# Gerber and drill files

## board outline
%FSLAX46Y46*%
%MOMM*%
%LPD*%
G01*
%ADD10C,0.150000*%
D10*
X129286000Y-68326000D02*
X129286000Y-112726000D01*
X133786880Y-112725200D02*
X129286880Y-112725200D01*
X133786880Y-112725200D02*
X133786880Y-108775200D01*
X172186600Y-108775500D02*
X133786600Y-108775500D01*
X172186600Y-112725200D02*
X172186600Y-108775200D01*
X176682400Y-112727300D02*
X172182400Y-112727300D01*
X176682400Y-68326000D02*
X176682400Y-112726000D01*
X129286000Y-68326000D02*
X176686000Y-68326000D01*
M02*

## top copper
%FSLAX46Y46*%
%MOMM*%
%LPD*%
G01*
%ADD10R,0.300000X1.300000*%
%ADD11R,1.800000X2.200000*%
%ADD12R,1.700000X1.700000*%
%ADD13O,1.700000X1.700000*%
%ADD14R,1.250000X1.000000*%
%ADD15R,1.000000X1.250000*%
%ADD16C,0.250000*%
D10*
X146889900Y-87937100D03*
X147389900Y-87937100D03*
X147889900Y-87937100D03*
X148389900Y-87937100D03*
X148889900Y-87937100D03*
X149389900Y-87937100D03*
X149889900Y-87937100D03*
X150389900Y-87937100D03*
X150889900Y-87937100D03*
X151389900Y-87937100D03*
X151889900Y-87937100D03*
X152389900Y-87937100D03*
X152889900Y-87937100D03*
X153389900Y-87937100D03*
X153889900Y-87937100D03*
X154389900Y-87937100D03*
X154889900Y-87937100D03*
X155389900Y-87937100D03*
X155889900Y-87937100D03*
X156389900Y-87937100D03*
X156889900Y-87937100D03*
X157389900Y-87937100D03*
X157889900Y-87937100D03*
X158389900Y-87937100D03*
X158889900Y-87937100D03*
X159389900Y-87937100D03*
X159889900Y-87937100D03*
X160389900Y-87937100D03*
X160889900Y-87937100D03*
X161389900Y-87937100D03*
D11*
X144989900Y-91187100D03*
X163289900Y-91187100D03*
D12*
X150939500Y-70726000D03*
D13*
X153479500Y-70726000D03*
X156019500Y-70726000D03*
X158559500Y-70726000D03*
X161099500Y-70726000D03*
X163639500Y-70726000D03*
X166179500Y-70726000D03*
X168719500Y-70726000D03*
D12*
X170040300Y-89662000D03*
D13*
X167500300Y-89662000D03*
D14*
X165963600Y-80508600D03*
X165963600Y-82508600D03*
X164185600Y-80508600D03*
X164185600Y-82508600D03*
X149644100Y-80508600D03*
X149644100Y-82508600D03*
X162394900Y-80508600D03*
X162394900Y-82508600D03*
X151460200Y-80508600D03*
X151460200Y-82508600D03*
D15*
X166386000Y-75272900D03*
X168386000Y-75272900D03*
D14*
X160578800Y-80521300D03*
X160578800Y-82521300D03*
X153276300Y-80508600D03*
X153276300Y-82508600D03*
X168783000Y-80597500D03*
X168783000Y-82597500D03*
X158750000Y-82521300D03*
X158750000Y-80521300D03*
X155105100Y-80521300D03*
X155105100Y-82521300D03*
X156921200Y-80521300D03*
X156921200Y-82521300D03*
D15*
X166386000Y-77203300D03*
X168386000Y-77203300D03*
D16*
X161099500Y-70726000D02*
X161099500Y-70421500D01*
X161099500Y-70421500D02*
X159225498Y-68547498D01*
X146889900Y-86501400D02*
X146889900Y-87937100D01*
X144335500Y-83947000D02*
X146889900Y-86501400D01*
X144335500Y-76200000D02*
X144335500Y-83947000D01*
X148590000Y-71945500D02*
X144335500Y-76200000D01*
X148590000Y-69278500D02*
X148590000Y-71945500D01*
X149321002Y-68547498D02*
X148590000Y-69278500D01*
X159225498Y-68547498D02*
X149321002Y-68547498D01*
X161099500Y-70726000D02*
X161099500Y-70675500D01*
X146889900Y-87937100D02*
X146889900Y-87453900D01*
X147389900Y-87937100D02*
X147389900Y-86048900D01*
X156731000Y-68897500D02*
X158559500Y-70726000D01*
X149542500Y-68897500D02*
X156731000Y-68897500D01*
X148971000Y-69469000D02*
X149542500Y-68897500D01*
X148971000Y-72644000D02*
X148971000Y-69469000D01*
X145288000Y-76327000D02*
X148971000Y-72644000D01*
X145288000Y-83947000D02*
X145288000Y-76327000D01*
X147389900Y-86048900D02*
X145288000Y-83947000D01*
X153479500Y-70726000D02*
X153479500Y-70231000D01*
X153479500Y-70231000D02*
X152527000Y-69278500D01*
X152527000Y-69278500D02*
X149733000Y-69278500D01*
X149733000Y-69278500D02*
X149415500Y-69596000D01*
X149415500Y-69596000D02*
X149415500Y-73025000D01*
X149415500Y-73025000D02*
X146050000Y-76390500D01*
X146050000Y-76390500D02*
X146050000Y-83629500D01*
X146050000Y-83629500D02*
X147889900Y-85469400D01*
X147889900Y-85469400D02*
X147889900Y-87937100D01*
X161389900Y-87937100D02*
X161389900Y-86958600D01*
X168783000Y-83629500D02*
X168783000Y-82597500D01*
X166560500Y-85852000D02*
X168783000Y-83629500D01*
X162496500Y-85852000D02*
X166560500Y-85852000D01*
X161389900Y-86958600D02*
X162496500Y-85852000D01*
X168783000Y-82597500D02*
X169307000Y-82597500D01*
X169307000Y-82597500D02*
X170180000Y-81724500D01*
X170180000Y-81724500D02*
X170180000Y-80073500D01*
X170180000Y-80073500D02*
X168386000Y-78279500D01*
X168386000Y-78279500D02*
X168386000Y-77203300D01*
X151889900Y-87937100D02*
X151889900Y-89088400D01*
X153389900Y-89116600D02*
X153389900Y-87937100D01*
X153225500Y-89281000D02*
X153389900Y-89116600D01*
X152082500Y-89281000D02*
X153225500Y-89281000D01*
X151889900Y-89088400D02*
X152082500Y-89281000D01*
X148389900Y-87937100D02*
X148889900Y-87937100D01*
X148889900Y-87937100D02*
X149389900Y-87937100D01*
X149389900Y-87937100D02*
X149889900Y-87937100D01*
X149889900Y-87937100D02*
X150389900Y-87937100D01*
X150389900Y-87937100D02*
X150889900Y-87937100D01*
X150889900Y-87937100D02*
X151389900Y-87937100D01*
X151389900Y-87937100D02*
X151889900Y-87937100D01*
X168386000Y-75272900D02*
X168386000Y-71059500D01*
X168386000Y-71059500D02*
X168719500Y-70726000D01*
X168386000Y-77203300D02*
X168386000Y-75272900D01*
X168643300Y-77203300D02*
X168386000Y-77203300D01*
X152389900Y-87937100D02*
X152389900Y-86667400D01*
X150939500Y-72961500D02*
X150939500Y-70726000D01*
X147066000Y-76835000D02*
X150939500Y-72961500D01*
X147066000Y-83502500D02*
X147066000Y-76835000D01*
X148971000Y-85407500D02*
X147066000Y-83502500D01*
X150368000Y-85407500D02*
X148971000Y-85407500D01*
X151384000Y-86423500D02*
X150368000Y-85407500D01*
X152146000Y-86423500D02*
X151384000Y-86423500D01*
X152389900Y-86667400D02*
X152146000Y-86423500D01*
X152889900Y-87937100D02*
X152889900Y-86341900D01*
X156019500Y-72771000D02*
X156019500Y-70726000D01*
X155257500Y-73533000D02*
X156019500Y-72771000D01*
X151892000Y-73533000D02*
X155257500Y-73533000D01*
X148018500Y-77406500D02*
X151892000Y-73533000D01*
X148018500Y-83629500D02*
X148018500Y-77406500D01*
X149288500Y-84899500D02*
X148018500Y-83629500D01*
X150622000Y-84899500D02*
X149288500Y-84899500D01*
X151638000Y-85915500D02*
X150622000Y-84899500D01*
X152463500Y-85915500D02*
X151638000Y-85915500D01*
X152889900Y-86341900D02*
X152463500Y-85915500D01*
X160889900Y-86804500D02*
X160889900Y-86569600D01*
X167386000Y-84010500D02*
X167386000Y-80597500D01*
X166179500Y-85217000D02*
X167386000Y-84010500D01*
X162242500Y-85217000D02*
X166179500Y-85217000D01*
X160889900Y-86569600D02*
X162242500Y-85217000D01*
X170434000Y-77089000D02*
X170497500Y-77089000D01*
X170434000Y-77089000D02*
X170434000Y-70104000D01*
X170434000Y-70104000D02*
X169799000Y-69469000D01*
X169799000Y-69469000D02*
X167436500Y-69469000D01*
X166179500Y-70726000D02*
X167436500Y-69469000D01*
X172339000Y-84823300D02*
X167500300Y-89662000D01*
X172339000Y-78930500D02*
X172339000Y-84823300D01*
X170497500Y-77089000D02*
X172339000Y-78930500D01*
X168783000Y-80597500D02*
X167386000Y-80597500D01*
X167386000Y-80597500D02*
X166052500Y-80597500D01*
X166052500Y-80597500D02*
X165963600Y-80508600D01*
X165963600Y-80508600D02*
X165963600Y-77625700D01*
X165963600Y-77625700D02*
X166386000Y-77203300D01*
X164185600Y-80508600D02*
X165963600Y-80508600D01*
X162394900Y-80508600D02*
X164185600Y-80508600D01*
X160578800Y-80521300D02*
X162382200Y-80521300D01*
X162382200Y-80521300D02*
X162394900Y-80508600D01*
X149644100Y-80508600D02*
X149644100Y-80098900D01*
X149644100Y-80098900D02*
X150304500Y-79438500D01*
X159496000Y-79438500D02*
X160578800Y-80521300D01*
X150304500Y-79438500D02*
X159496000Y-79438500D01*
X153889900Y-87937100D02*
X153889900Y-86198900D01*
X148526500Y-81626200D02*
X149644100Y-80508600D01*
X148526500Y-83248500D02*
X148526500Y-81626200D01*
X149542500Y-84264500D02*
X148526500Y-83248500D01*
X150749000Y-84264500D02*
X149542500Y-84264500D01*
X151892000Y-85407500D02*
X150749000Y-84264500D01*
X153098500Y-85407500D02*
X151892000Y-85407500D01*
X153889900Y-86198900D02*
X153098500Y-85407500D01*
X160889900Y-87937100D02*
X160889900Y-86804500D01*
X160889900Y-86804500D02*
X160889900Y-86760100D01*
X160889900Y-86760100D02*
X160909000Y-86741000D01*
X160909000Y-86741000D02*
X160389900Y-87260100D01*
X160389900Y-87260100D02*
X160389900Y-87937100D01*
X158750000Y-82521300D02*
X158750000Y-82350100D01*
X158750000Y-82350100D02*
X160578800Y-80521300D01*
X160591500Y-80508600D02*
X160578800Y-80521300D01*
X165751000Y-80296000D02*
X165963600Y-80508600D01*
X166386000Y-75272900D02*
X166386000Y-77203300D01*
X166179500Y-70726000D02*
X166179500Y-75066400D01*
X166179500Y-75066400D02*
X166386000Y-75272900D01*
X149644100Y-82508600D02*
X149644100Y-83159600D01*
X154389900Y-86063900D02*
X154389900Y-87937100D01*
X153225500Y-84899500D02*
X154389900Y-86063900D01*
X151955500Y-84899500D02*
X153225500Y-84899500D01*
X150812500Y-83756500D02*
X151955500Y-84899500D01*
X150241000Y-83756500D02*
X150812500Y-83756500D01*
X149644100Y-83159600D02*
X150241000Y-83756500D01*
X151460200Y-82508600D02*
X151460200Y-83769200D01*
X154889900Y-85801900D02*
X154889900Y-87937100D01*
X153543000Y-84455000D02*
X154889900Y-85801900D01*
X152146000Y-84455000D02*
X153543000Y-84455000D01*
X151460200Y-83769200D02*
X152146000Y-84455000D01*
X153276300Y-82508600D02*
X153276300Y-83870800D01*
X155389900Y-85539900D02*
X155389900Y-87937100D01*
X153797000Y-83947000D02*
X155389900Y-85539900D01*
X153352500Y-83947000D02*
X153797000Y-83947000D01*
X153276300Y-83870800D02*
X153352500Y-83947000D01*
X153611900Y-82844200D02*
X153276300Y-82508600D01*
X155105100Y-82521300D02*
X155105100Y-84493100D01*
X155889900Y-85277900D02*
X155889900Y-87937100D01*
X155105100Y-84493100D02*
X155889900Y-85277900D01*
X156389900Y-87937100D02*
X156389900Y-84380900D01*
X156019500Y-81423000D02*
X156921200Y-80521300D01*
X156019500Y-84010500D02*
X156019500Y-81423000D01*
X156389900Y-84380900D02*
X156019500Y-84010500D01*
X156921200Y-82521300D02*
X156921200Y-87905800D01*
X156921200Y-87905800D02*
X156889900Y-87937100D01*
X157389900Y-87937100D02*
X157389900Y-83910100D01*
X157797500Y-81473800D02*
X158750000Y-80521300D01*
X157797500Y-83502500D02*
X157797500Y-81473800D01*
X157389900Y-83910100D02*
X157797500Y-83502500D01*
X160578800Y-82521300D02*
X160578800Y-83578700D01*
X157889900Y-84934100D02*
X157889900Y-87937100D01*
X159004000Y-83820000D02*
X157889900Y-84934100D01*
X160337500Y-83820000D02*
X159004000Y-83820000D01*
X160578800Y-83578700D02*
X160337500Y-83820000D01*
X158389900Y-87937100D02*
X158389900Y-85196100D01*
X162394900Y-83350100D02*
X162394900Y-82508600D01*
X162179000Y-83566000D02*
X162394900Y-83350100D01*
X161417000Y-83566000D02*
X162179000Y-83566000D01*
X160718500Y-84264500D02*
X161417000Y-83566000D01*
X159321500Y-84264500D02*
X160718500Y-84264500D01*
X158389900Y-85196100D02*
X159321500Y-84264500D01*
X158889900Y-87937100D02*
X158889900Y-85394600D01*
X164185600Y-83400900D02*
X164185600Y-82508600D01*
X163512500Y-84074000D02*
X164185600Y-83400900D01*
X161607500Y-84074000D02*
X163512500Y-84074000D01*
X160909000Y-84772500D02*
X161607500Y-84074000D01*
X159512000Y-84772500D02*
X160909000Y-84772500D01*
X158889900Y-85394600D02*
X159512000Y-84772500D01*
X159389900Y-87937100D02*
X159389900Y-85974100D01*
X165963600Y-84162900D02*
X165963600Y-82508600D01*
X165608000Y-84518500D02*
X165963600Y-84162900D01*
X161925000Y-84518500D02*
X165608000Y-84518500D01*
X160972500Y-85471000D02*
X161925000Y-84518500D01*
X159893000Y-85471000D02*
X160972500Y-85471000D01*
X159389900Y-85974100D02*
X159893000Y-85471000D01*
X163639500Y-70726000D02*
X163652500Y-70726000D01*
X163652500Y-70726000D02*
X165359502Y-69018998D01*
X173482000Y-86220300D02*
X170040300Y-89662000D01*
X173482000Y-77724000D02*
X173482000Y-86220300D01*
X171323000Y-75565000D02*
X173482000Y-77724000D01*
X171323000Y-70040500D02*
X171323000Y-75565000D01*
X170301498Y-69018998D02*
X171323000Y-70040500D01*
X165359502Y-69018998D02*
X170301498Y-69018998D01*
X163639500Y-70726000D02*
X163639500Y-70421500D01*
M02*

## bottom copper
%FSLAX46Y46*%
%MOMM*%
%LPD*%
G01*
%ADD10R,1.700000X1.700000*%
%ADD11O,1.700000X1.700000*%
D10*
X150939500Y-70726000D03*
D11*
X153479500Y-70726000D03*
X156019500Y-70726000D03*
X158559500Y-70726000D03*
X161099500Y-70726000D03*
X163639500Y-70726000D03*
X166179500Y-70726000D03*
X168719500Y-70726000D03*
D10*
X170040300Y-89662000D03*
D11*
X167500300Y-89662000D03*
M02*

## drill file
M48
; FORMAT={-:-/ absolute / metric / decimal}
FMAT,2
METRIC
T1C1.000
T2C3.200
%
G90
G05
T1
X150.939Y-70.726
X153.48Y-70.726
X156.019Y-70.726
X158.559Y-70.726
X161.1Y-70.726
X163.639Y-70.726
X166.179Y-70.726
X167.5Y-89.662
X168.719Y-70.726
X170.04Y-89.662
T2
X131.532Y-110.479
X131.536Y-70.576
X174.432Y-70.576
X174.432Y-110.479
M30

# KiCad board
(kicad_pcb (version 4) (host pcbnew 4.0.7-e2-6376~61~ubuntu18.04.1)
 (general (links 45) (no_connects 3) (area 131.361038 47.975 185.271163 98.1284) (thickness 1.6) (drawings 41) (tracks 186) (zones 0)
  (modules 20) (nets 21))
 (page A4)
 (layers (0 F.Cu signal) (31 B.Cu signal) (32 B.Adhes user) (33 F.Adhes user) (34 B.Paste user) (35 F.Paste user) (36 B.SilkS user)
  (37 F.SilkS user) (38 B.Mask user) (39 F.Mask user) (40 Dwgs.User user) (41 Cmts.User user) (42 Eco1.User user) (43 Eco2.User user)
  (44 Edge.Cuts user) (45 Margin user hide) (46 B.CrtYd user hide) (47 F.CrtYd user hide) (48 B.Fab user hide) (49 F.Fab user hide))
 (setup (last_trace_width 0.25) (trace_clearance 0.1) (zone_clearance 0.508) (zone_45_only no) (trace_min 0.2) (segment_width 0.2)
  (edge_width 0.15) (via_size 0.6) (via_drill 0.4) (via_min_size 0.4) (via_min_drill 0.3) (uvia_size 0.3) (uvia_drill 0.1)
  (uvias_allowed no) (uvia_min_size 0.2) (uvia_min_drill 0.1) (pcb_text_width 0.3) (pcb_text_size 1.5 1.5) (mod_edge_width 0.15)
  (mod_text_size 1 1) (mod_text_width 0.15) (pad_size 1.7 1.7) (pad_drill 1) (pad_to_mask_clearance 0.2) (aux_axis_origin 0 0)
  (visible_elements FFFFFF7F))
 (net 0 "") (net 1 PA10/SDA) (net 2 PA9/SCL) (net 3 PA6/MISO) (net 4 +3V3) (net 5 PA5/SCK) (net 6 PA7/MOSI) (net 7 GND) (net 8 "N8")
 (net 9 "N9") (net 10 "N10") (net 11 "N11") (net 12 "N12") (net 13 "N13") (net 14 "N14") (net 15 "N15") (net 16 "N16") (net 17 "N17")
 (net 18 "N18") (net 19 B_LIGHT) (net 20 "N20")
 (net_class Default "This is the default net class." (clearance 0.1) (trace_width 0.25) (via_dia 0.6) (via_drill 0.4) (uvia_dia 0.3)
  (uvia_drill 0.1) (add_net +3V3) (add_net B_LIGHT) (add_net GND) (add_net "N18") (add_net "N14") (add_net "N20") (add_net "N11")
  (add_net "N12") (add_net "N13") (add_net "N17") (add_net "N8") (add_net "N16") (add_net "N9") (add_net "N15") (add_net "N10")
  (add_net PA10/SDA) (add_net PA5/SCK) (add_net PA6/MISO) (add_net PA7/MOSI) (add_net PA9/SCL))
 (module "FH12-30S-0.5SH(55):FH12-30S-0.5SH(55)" (layer F.Cu) (at 154.1399 88.4301)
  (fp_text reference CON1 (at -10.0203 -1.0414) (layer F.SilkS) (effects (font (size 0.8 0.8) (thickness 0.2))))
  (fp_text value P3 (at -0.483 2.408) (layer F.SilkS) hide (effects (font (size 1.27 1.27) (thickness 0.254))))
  (pad 1 smd rect (at -7.25 -0.493) (size 0.3 1.3) (layers F.Cu F.Paste F.Mask) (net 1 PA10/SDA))
  (pad 2 smd rect (at -6.75 -0.493) (size 0.3 1.3) (layers F.Cu F.Paste F.Mask) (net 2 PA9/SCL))
  (pad 3 smd rect (at -6.25 -0.493) (size 0.3 1.3) (layers F.Cu F.Paste F.Mask) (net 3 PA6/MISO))
  (pad 4 smd rect (at -5.75 -0.493) (size 0.3 1.3) (layers F.Cu F.Paste F.Mask) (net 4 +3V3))
  (pad 5 smd rect (at -5.25 -0.493) (size 0.3 1.3) (layers F.Cu F.Paste F.Mask) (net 4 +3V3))
  (pad 6 smd rect (at -4.75 -0.493) (size 0.3 1.3) (layers F.Cu F.Paste F.Mask) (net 4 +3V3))
  (pad 7 smd rect (at -4.25 -0.493) (size 0.3 1.3) (layers F.Cu F.Paste F.Mask) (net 4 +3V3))
  (pad 8 smd rect (at -3.75 -0.493) (size 0.3 1.3) (layers F.Cu F.Paste F.Mask) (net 4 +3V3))
  (pad 9 smd rect (at -3.25 -0.493) (size 0.3 1.3) (layers F.Cu F.Paste F.Mask) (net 4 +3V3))
  (pad 10 smd rect (at -2.75 -0.493) (size 0.3 1.3) (layers F.Cu F.Paste F.Mask) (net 4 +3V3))
  (pad 11 smd rect (at -2.25 -0.493) (size 0.3 1.3) (layers F.Cu F.Paste F.Mask) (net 4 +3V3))
  (pad 12 smd rect (at -1.75 -0.493) (size 0.3 1.3) (layers F.Cu F.Paste F.Mask) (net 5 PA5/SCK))
  (pad 13 smd rect (at -1.25 -0.493) (size 0.3 1.3) (layers F.Cu F.Paste F.Mask) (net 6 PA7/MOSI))
  (pad 14 smd rect (at -0.75 -0.493) (size 0.3 1.3) (layers F.Cu F.Paste F.Mask) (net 4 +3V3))
  (pad 15 smd rect (at -0.25 -0.493) (size 0.3 1.3) (layers F.Cu F.Paste F.Mask) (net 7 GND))
  (pad 16 smd rect (at 0.25 -0.493) (size 0.3 1.3) (layers F.Cu F.Paste F.Mask) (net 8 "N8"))
  (pad 17 smd rect (at 0.75 -0.493) (size 0.3 1.3) (layers F.Cu F.Paste F.Mask) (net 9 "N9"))
  (pad 18 smd rect (at 1.25 -0.493) (size 0.3 1.3) (layers F.Cu F.Paste F.Mask) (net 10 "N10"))
  (pad 19 smd rect (at 1.75 -0.493) (size 0.3 1.3) (layers F.Cu F.Paste F.Mask) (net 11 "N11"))
  (pad 20 smd rect (at 2.25 -0.493) (size 0.3 1.3) (layers F.Cu F.Paste F.Mask) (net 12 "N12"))
  (pad 21 smd rect (at 2.75 -0.493) (size 0.3 1.3) (layers F.Cu F.Paste F.Mask) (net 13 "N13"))
  (pad 22 smd rect (at 3.25 -0.493) (size 0.3 1.3) (layers F.Cu F.Paste F.Mask) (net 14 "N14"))
  (pad 23 smd rect (at 3.75 -0.493) (size 0.3 1.3) (layers F.Cu F.Paste F.Mask) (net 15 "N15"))
  (pad 24 smd rect (at 4.25 -0.493) (size 0.3 1.3) (layers F.Cu F.Paste F.Mask) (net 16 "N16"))
  (pad 25 smd rect (at 4.75 -0.493) (size 0.3 1.3) (layers F.Cu F.Paste F.Mask) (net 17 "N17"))
  (pad 26 smd rect (at 5.25 -0.493) (size 0.3 1.3) (layers F.Cu F.Paste F.Mask) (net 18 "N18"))
  (pad 27 smd rect (at 5.75 -0.493) (size 0.3 1.3) (layers F.Cu F.Paste F.Mask))
  (pad 28 smd rect (at 6.25 -0.493) (size 0.3 1.3) (layers F.Cu F.Paste F.Mask) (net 7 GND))
  (pad 29 smd rect (at 6.75 -0.493) (size 0.3 1.3) (layers F.Cu F.Paste F.Mask) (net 7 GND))
  (pad 30 smd rect (at 7.25 -0.493) (size 0.3 1.3) (layers F.Cu F.Paste F.Mask) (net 4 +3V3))
  (pad 31 smd rect (at -9.15 2.757) (size 1.8 2.2) (layers F.Cu F.Paste F.Mask))
  (pad 32 smd rect (at 9.15 2.757) (size 1.8 2.2) (layers F.Cu F.Paste F.Mask)))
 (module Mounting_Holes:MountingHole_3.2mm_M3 (layer F.Cu) (at 174.4324 110.4794)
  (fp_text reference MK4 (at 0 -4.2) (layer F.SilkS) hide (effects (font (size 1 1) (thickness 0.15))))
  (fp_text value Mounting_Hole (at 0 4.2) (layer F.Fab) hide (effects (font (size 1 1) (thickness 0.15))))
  (pad 1 np_thru_hole circle (at 0 0) (size 3.2 3.2) (drill 3.2) (layers *.Cu *.Mask)))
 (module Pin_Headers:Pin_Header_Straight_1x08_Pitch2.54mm (layer F.Cu) (at 150.9395 70.726 90)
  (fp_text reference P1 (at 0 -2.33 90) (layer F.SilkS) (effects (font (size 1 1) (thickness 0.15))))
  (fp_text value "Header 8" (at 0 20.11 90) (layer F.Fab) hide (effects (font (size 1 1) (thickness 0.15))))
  (pad 1 thru_hole rect (at 0 0 90) (size 1.7 1.7) (drill 1) (layers *.Cu *.Mask) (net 5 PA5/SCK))
  (pad 2 thru_hole oval (at 0 2.54 90) (size 1.7 1.7) (drill 1) (layers *.Cu *.Mask) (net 3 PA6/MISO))
  (pad 3 thru_hole oval (at 0 5.08 90) (size 1.7 1.7) (drill 1) (layers *.Cu *.Mask) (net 6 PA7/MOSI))
  (pad 4 thru_hole oval (at 0 7.62 90) (size 1.7 1.7) (drill 1) (layers *.Cu *.Mask) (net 2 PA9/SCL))
  (pad 5 thru_hole oval (at 0 10.16 90) (size 1.7 1.7) (drill 1) (layers *.Cu *.Mask) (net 1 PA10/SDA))
  (pad 6 thru_hole oval (at 0 12.7 90) (size 1.7 1.7) (drill 1) (layers *.Cu *.Mask) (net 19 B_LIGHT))
  (pad 7 thru_hole oval (at 0 15.24 90) (size 1.7 1.7) (drill 1) (layers *.Cu *.Mask) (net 7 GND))
  (pad 8 thru_hole oval (at 0 17.78 90) (size 1.7 1.7) (drill 1) (layers *.Cu *.Mask) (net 4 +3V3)))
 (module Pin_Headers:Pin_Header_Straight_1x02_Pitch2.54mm (layer F.Cu) (at 170.0403 89.662 270)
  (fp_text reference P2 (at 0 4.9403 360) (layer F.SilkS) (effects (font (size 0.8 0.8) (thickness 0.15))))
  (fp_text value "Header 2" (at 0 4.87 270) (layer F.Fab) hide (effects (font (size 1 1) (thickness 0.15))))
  (pad 1 thru_hole rect (at 0 0 270) (size 1.7 1.7) (drill 1) (layers *.Cu *.Mask) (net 19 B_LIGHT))
  (pad 2 thru_hole oval (at 0 2.54 270) (size 1.7 1.7) (drill 1) (layers *.Cu *.Mask) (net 7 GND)))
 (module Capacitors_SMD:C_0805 (layer F.Cu) (at 165.9636 81.5086 270)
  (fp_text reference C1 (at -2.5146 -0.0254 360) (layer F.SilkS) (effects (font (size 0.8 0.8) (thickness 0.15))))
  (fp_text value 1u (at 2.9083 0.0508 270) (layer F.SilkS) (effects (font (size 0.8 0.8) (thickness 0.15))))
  (pad 1 smd rect (at -1 0 270) (size 1 1.25) (layers F.Cu F.Paste F.Mask) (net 7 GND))
  (pad 2 smd rect (at 1 0 270) (size 1 1.25) (layers F.Cu F.Paste F.Mask) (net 18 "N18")))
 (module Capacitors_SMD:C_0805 (layer F.Cu) (at 164.1856 81.5086 270)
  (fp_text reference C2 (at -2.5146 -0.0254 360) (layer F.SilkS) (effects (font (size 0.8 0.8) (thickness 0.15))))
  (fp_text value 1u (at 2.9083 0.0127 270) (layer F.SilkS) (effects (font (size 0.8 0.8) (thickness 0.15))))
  (pad 1 smd rect (at -1 0 270) (size 1 1.25) (layers F.Cu F.Paste F.Mask) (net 7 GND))
  (pad 2 smd rect (at 1 0 270) (size 1 1.25) (layers F.Cu F.Paste F.Mask) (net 17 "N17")))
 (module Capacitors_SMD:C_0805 (layer F.Cu) (at 149.6441 81.5086 270)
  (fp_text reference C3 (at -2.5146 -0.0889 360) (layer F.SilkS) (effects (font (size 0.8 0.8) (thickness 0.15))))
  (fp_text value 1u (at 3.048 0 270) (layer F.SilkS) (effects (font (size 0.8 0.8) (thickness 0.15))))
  (pad 1 smd rect (at -1 0 270) (size 1 1.25) (layers F.Cu F.Paste F.Mask) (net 7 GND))
  (pad 2 smd rect (at 1 0 270) (size 1 1.25) (layers F.Cu F.Paste F.Mask) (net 8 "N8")))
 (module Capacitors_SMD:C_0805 (layer F.Cu) (at 162.3949 81.5086 270)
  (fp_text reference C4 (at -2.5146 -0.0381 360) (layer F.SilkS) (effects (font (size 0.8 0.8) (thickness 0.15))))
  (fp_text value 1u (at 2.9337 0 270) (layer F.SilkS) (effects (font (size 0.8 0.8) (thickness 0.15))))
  (pad 1 smd rect (at -1 0 270) (size 1 1.25) (layers F.Cu F.Paste F.Mask) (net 7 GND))
  (pad 2 smd rect (at 1 0 270) (size 1 1.25) (layers F.Cu F.Paste F.Mask) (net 16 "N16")))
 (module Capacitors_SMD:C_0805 (layer F.Cu) (at 151.4602 81.5086 270)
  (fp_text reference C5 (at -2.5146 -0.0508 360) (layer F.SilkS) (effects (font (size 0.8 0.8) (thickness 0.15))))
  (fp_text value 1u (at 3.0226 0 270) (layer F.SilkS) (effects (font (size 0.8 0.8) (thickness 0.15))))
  (pad 1 smd rect (at -1 0 270) (size 1 1.25) (layers F.Cu F.Paste F.Mask) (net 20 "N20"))
  (pad 2 smd rect (at 1 0 270) (size 1 1.25) (layers F.Cu F.Paste F.Mask) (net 9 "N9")))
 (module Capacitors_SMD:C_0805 (layer F.Cu) (at 167.386 75.2729)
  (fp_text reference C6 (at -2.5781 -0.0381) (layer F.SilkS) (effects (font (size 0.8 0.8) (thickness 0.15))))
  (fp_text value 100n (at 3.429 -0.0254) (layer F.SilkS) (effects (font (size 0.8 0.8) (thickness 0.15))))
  (pad 1 smd rect (at -1 0) (size 1 1.25) (layers F.Cu F.Paste F.Mask) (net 7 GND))
  (pad 2 smd rect (at 1 0) (size 1 1.25) (layers F.Cu F.Paste F.Mask) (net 4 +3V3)))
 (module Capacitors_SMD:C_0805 (layer F.Cu) (at 160.5788 81.5213 270)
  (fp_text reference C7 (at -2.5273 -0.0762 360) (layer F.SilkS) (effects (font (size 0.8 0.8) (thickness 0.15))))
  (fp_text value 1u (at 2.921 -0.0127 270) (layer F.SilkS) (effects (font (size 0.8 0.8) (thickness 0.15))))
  (pad 1 smd rect (at -1 0 270) (size 1 1.25) (layers F.Cu F.Paste F.Mask) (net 7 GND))
  (pad 2 smd rect (at 1 0 270) (size 1 1.25) (layers F.Cu F.Paste F.Mask) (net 15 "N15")))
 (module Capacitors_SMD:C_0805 (layer F.Cu) (at 153.2763 81.5086 270)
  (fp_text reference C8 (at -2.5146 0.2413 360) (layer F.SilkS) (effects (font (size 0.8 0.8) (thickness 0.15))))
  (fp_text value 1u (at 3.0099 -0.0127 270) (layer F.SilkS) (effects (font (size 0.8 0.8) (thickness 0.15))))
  (pad 1 smd rect (at -1 0 270) (size 1 1.25) (layers F.Cu F.Paste F.Mask) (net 20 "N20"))
  (pad 2 smd rect (at 1 0 270) (size 1 1.25) (layers F.Cu F.Paste F.Mask) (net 10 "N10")))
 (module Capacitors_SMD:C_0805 (layer F.Cu) (at 168.783 81.5975 270)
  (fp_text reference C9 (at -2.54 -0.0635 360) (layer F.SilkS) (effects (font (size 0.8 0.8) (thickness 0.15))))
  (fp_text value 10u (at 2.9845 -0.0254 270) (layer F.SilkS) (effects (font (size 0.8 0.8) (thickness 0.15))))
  (pad 1 smd rect (at -1 0 270) (size 1 1.25) (layers F.Cu F.Paste F.Mask) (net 7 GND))
  (pad 2 smd rect (at 1 0 270) (size 1 1.25) (layers F.Cu F.Paste F.Mask) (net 4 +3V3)))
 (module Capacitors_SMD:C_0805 (layer F.Cu) (at 158.75 81.5213 90)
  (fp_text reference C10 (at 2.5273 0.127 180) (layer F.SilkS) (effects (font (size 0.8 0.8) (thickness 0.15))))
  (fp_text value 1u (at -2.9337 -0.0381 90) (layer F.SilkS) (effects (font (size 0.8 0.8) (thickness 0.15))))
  (pad 1 smd rect (at -1 0 90) (size 1 1.25) (layers F.Cu F.Paste F.Mask) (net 7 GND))
  (pad 2 smd rect (at 1 0 90) (size 1 1.25) (layers F.Cu F.Paste F.Mask) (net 14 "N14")))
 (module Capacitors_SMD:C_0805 (layer F.Cu) (at 155.1051 81.5213 270)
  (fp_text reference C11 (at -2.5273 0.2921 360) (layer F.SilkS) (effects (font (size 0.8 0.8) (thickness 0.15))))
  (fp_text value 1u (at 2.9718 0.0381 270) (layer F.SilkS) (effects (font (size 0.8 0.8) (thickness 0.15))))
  (pad 1 smd rect (at -1 0 270) (size 1 1.25) (layers F.Cu F.Paste F.Mask) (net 20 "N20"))
  (pad 2 smd rect (at 1 0 270) (size 1 1.25) (layers F.Cu F.Paste F.Mask) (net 11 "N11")))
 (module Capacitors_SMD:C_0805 (layer F.Cu) (at 156.9212 81.5213 270)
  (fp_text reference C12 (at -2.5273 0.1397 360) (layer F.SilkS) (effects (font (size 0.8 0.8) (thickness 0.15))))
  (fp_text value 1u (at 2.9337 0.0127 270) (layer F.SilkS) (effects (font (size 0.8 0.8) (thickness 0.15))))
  (pad 1 smd rect (at -1 0 270) (size 1 1.25) (layers F.Cu F.Paste F.Mask) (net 12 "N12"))
  (pad 2 smd rect (at 1 0 270) (size 1 1.25) (layers F.Cu F.Paste F.Mask) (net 13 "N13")))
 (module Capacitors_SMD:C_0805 (layer F.Cu) (at 167.386 77.2033)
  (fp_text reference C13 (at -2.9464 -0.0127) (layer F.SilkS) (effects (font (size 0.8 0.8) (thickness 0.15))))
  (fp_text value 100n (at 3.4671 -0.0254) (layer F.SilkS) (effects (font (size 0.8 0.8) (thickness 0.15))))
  (pad 1 smd rect (at -1 0) (size 1 1.25) (layers F.Cu F.Paste F.Mask) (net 7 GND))
  (pad 2 smd rect (at 1 0) (size 1 1.25) (layers F.Cu F.Paste F.Mask) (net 4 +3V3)))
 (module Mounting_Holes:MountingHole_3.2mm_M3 (layer F.Cu) (at 131.536 70.576)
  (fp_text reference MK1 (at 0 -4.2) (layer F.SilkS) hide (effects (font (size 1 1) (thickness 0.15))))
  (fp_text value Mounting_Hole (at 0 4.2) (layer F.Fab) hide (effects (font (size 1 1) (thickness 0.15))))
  (pad 1 np_thru_hole circle (at 0 0) (size 3.2 3.2) (drill 3.2) (layers *.Cu *.Mask)))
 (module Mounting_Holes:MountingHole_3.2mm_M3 (layer F.Cu) (at 174.4324 70.576)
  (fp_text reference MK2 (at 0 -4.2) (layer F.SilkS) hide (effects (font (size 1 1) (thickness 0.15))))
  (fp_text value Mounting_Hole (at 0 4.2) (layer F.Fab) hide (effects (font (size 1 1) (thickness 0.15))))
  (pad 1 np_thru_hole circle (at 0 0) (size 3.2 3.2) (drill 3.2) (layers *.Cu *.Mask)))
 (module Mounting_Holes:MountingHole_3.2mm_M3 (layer F.Cu) (at 131.5318 110.4794)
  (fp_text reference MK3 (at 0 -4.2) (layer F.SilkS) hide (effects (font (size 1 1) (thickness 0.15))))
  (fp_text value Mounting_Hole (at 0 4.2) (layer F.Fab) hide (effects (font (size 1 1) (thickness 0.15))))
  (pad 1 np_thru_hole circle (at 0 0) (size 3.2 3.2) (drill 3.2) (layers *.Cu *.Mask)))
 (gr_line (start 129.286 68.326) (end 129.286 112.726) (angle 90) (layer Edge.Cuts) (width 0.15))
 (gr_line (start 133.78688 112.7252) (end 129.28688 112.7252) (angle 90) (layer Edge.Cuts) (width 0.15))
 (gr_line (start 133.78688 112.7252) (end 133.78688 108.7752) (angle 90) (layer Edge.Cuts) (width 0.15))
 (gr_line (start 172.1866 108.7755) (end 133.7866 108.7755) (angle 90) (layer Edge.Cuts) (width 0.15))
 (gr_line (start 172.1866 112.7252) (end 172.1866 108.7752) (angle 90) (layer Edge.Cuts) (width 0.15))
 (gr_line (start 176.6824 112.7273) (end 172.1824 112.7273) (angle 90) (layer Edge.Cuts) (width 0.15))
 (gr_line (start 176.6824 68.326) (end 176.6824 112.726) (angle 90) (layer Edge.Cuts) (width 0.15))
 (gr_line (start 129.286 68.326) (end 176.686 68.326) (angle 90) (layer Edge.Cuts) (width 0.15))
 (segment (start 161.0995 70.726) (end 161.0995 70.4215) (width 0.25) (layer F.Cu) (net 1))
 (segment (start 161.0995 70.4215) (end 159.225498 68.547498) (width 0.25) (layer F.Cu) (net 1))
 (segment (start 146.8899 86.5014) (end 146.8899 87.9371) (width 0.25) (layer F.Cu) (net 1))
 (segment (start 144.3355 83.947) (end 146.8899 86.5014) (width 0.25) (layer F.Cu) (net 1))
 (segment (start 144.3355 76.2) (end 144.3355 83.947) (width 0.25) (layer F.Cu) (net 1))
 (segment (start 148.59 71.9455) (end 144.3355 76.2) (width 0.25) (layer F.Cu) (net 1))
 (segment (start 148.59 69.2785) (end 148.59 71.9455) (width 0.25) (layer F.Cu) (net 1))
 (segment (start 149.321002 68.547498) (end 148.59 69.2785) (width 0.25) (layer F.Cu) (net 1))
 (segment (start 159.225498 68.547498) (end 149.321002 68.547498) (width 0.25) (layer F.Cu) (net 1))
 (segment (start 161.0995 70.726) (end 161.0995 70.6755) (width 0.25) (layer F.Cu) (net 1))
 (segment (start 146.8899 87.9371) (end 146.8899 87.4539) (width 0.25) (layer F.Cu) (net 1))
 (segment (start 147.3899 87.9371) (end 147.3899 86.0489) (width 0.25) (layer F.Cu) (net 2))
 (segment (start 156.731 68.8975) (end 158.5595 70.726) (width 0.25) (layer F.Cu) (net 2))
 (segment (start 149.5425 68.8975) (end 156.731 68.8975) (width 0.25) (layer F.Cu) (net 2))
 (segment (start 148.971 69.469) (end 149.5425 68.8975) (width 0.25) (layer F.Cu) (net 2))
 (segment (start 148.971 72.644) (end 148.971 69.469) (width 0.25) (layer F.Cu) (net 2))
 (segment (start 145.288 76.327) (end 148.971 72.644) (width 0.25) (layer F.Cu) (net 2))
 (segment (start 145.288 83.947) (end 145.288 76.327) (width 0.25) (layer F.Cu) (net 2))
 (segment (start 147.3899 86.0489) (end 145.288 83.947) (width 0.25) (layer F.Cu) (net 2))
 (segment (start 153.4795 70.726) (end 153.4795 70.231) (width 0.25) (layer F.Cu) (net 3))
 (segment (start 153.4795 70.231) (end 152.527 69.2785) (width 0.25) (layer F.Cu) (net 3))
 (segment (start 152.527 69.2785) (end 149.733 69.2785) (width 0.25) (layer F.Cu) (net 3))
 (segment (start 149.733 69.2785) (end 149.4155 69.596) (width 0.25) (layer F.Cu) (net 3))
 (segment (start 149.4155 69.596) (end 149.4155 73.025) (width 0.25) (layer F.Cu) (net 3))
 (segment (start 149.4155 73.025) (end 146.05 76.3905) (width 0.25) (layer F.Cu) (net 3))
 (segment (start 146.05 76.3905) (end 146.05 83.6295) (width 0.25) (layer F.Cu) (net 3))
 (segment (start 146.05 83.6295) (end 147.8899 85.4694) (width 0.25) (layer F.Cu) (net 3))
 (segment (start 147.8899 85.4694) (end 147.8899 87.9371) (width 0.25) (layer F.Cu) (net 3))
 (segment (start 161.3899 87.9371) (end 161.3899 86.9586) (width 0.25) (layer F.Cu) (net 4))
 (segment (start 168.783 83.6295) (end 168.783 82.5975) (width 0.25) (layer F.Cu) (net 4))
 (segment (start 166.5605 85.852) (end 168.783 83.6295) (width 0.25) (layer F.Cu) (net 4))
 (segment (start 162.4965 85.852) (end 166.5605 85.852) (width 0.25) (layer F.Cu) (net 4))
 (segment (start 161.3899 86.9586) (end 162.4965 85.852) (width 0.25) (layer F.Cu) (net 4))
 (segment (start 168.783 82.5975) (end 169.307 82.5975) (width 0.25) (layer F.Cu) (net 4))
 (segment (start 169.307 82.5975) (end 170.18 81.7245) (width 0.25) (layer F.Cu) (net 4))
 (segment (start 170.18 81.7245) (end 170.18 80.0735) (width 0.25) (layer F.Cu) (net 4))
 (segment (start 170.18 80.0735) (end 168.386 78.2795) (width 0.25) (layer F.Cu) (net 4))
 (segment (start 168.386 78.2795) (end 168.386 77.2033) (width 0.25) (layer F.Cu) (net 4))
 (segment (start 151.8899 87.9371) (end 151.8899 89.0884) (width 0.25) (layer F.Cu) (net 4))
 (segment (start 153.3899 89.1166) (end 153.3899 87.9371) (width 0.25) (layer F.Cu) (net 4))
 (segment (start 153.2255 89.281) (end 153.3899 89.1166) (width 0.25) (layer F.Cu) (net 4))
 (segment (start 152.0825 89.281) (end 153.2255 89.281) (width 0.25) (layer F.Cu) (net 4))
 (segment (start 151.8899 89.0884) (end 152.0825 89.281) (width 0.25) (layer F.Cu) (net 4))
 (segment (start 148.3899 87.9371) (end 148.8899 87.9371) (width 0.25) (layer F.Cu) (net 4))
 (segment (start 148.8899 87.9371) (end 149.3899 87.9371) (width 0.25) (layer F.Cu) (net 4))
 (segment (start 149.3899 87.9371) (end 149.8899 87.9371) (width 0.25) (layer F.Cu) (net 4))
 (segment (start 149.8899 87.9371) (end 150.3899 87.9371) (width 0.25) (layer F.Cu) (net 4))
 (segment (start 150.3899 87.9371) (end 150.8899 87.9371) (width 0.25) (layer F.Cu) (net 4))
 (segment (start 150.8899 87.9371) (end 151.3899 87.9371) (width 0.25) (layer F.Cu) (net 4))
 (segment (start 151.3899 87.9371) (end 151.8899 87.9371) (width 0.25) (layer F.Cu) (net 4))
 (segment (start 168.386 75.2729) (end 168.386 71.0595) (width 0.25) (layer F.Cu) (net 4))
 (segment (start 168.386 71.0595) (end 168.7195 70.726) (width 0.25) (layer F.Cu) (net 4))
 (segment (start 168.386 77.2033) (end 168.386 75.2729) (width 0.25) (layer F.Cu) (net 4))
 (segment (start 168.6433 77.2033) (end 168.386 77.2033) (width 0.25) (layer F.Cu) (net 4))
 (segment (start 152.3899 87.9371) (end 152.3899 86.6674) (width 0.25) (layer F.Cu) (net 5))
 (segment (start 150.9395 72.9615) (end 150.9395 70.726) (width 0.25) (layer F.Cu) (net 5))
 (segment (start 147.066 76.835) (end 150.9395 72.9615) (width 0.25) (layer F.Cu) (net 5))
 (segment (start 147.066 83.5025) (end 147.066 76.835) (width 0.25) (layer F.Cu) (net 5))
 (segment (start 148.971 85.4075) (end 147.066 83.5025) (width 0.25) (layer F.Cu) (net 5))
 (segment (start 150.368 85.4075) (end 148.971 85.4075) (width 0.25) (layer F.Cu) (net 5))
 (segment (start 151.384 86.4235) (end 150.368 85.4075) (width 0.25) (layer F.Cu) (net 5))
 (segment (start 152.146 86.4235) (end 151.384 86.4235) (width 0.25) (layer F.Cu) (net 5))
 (segment (start 152.3899 86.6674) (end 152.146 86.4235) (width 0.25) (layer F.Cu) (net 5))
 (segment (start 152.8899 87.9371) (end 152.8899 86.3419) (width 0.25) (layer F.Cu) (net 6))
 (segment (start 156.0195 72.771) (end 156.0195 70.726) (width 0.25) (layer F.Cu) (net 6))
 (segment (start 155.2575 73.533) (end 156.0195 72.771) (width 0.25) (layer F.Cu) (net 6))
 (segment (start 151.892 73.533) (end 155.2575 73.533) (width 0.25) (layer F.Cu) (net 6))
 (segment (start 148.0185 77.4065) (end 151.892 73.533) (width 0.25) (layer F.Cu) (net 6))
 (segment (start 148.0185 83.6295) (end 148.0185 77.4065) (width 0.25) (layer F.Cu) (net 6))
 (segment (start 149.2885 84.8995) (end 148.0185 83.6295) (width 0.25) (layer F.Cu) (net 6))
 (segment (start 150.622 84.8995) (end 149.2885 84.8995) (width 0.25) (layer F.Cu) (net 6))
 (segment (start 151.638 85.9155) (end 150.622 84.8995) (width 0.25) (layer F.Cu) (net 6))
 (segment (start 152.4635 85.9155) (end 151.638 85.9155) (width 0.25) (layer F.Cu) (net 6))
 (segment (start 152.8899 86.3419) (end 152.4635 85.9155) (width 0.25) (layer F.Cu) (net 6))
 (segment (start 160.8899 86.8045) (end 160.8899 86.5696) (width 0.25) (layer F.Cu) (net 7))
 (segment (start 167.386 84.0105) (end 167.386 80.5975) (width 0.25) (layer F.Cu) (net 7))
 (segment (start 166.1795 85.217) (end 167.386 84.0105) (width 0.25) (layer F.Cu) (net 7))
 (segment (start 162.2425 85.217) (end 166.1795 85.217) (width 0.25) (layer F.Cu) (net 7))
 (segment (start 160.8899 86.5696) (end 162.2425 85.217) (width 0.25) (layer F.Cu) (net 7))
 (segment (start 170.434 77.089) (end 170.4975 77.089) (width 0.25) (layer F.Cu) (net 7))
 (segment (start 170.434 77.089) (end 170.434 70.104) (width 0.25) (layer F.Cu) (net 7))
 (segment (start 170.434 70.104) (end 169.799 69.469) (width 0.25) (layer F.Cu) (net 7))
 (segment (start 169.799 69.469) (end 167.4365 69.469) (width 0.25) (layer F.Cu) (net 7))
 (segment (start 166.1795 70.726) (end 167.4365 69.469) (width 0.25) (layer F.Cu) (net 7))
 (segment (start 172.339 84.8233) (end 167.5003 89.662) (width 0.25) (layer F.Cu) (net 7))
 (segment (start 172.339 78.9305) (end 172.339 84.8233) (width 0.25) (layer F.Cu) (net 7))
 (segment (start 170.4975 77.089) (end 172.339 78.9305) (width 0.25) (layer F.Cu) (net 7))
 (segment (start 168.783 80.5975) (end 167.386 80.5975) (width 0.25) (layer F.Cu) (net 7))
 (segment (start 167.386 80.5975) (end 166.0525 80.5975) (width 0.25) (layer F.Cu) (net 7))
 (segment (start 166.0525 80.5975) (end 165.9636 80.5086) (width 0.25) (layer F.Cu) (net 7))
 (segment (start 165.9636 80.5086) (end 165.9636 77.6257) (width 0.25) (layer F.Cu) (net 7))
 (segment (start 165.9636 77.6257) (end 166.386 77.2033) (width 0.25) (layer F.Cu) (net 7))
 (segment (start 164.1856 80.5086) (end 165.9636 80.5086) (width 0.25) (layer F.Cu) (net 7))
 (segment (start 162.3949 80.5086) (end 164.1856 80.5086) (width 0.25) (layer F.Cu) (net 7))
 (segment (start 160.5788 80.5213) (end 162.3822 80.5213) (width 0.25) (layer F.Cu) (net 7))
 (segment (start 162.3822 80.5213) (end 162.3949 80.5086) (width 0.25) (layer F.Cu) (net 7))
 (segment (start 149.6441 80.5086) (end 149.6441 80.0989) (width 0.25) (layer F.Cu) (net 7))
 (segment (start 149.6441 80.0989) (end 150.3045 79.4385) (width 0.25) (layer F.Cu) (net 7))
 (segment (start 159.496 79.4385) (end 160.5788 80.5213) (width 0.25) (layer F.Cu) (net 7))
 (segment (start 150.3045 79.4385) (end 159.496 79.4385) (width 0.25) (layer F.Cu) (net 7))
 (segment (start 153.8899 87.9371) (end 153.8899 86.1989) (width 0.25) (layer F.Cu) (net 7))
 (segment (start 148.5265 81.6262) (end 149.6441 80.5086) (width 0.25) (layer F.Cu) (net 7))
 (segment (start 148.5265 83.2485) (end 148.5265 81.6262) (width 0.25) (layer F.Cu) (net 7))
 (segment (start 149.5425 84.2645) (end 148.5265 83.2485) (width 0.25) (layer F.Cu) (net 7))
 (segment (start 150.749 84.2645) (end 149.5425 84.2645) (width 0.25) (layer F.Cu) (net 7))
 (segment (start 151.892 85.4075) (end 150.749 84.2645) (width 0.25) (layer F.Cu) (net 7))
 (segment (start 153.0985 85.4075) (end 151.892 85.4075) (width 0.25) (layer F.Cu) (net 7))
 (segment (start 153.8899 86.1989) (end 153.0985 85.4075) (width 0.25) (layer F.Cu) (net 7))
 (segment (start 160.8899 87.9371) (end 160.8899 86.8045) (width 0.25) (layer F.Cu) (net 7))
 (segment (start 160.8899 86.8045) (end 160.8899 86.7601) (width 0.25) (layer F.Cu) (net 7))
 (segment (start 160.8899 86.7601) (end 160.909 86.741) (width 0.25) (layer F.Cu) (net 7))
 (segment (start 160.909 86.741) (end 160.3899 87.2601) (width 0.25) (layer F.Cu) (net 7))
 (segment (start 160.3899 87.2601) (end 160.3899 87.9371) (width 0.25) (layer F.Cu) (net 7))
 (segment (start 158.75 82.5213) (end 158.75 82.3501) (width 0.25) (layer F.Cu) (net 7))
 (segment (start 158.75 82.3501) (end 160.5788 80.5213) (width 0.25) (layer F.Cu) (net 7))
 (segment (start 160.5915 80.5086) (end 160.5788 80.5213) (width 0.25) (layer F.Cu) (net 7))
 (segment (start 165.751 80.296) (end 165.9636 80.5086) (width 0.25) (layer F.Cu) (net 7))
 (segment (start 166.386 75.2729) (end 166.386 77.2033) (width 0.25) (layer F.Cu) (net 7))
 (segment (start 166.1795 70.726) (end 166.1795 75.0664) (width 0.25) (layer F.Cu) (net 7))
 (segment (start 166.1795 75.0664) (end 166.386 75.2729) (width 0.25) (layer F.Cu) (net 7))
 (segment (start 149.6441 82.5086) (end 149.6441 83.1596) (width 0.25) (layer F.Cu) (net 8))
 (segment (start 154.3899 86.0639) (end 154.3899 87.9371) (width 0.25) (layer F.Cu) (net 8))
 (segment (start 153.2255 84.8995) (end 154.3899 86.0639) (width 0.25) (layer F.Cu) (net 8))
 (segment (start 151.9555 84.8995) (end 153.2255 84.8995) (width 0.25) (layer F.Cu) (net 8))
 (segment (start 150.8125 83.7565) (end 151.9555 84.8995) (width 0.25) (layer F.Cu) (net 8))
 (segment (start 150.241 83.7565) (end 150.8125 83.7565) (width 0.25) (layer F.Cu) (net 8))
 (segment (start 149.6441 83.1596) (end 150.241 83.7565) (width 0.25) (layer F.Cu) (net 8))
 (segment (start 151.4602 82.5086) (end 151.4602 83.7692) (width 0.25) (layer F.Cu) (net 9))
 (segment (start 154.8899 85.8019) (end 154.8899 87.9371) (width 0.25) (layer F.Cu) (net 9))
 (segment (start 153.543 84.455) (end 154.8899 85.8019) (width 0.25) (layer F.Cu) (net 9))
 (segment (start 152.146 84.455) (end 153.543 84.455) (width 0.25) (layer F.Cu) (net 9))
 (segment (start 151.4602 83.7692) (end 152.146 84.455) (width 0.25) (layer F.Cu) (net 9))
 (segment (start 153.2763 82.5086) (end 153.2763 83.8708) (width 0.25) (layer F.Cu) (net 10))
 (segment (start 155.3899 85.5399) (end 155.3899 87.9371) (width 0.25) (layer F.Cu) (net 10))
 (segment (start 153.797 83.947) (end 155.3899 85.5399) (width 0.25) (layer F.Cu) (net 10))
 (segment (start 153.3525 83.947) (end 153.797 83.947) (width 0.25) (layer F.Cu) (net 10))
 (segment (start 153.2763 83.8708) (end 153.3525 83.947) (width 0.25) (layer F.Cu) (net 10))
 (segment (start 153.6119 82.8442) (end 153.2763 82.5086) (width 0.25) (layer F.Cu) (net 10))
 (segment (start 155.1051 82.5213) (end 155.1051 84.4931) (width 0.25) (layer F.Cu) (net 11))
 (segment (start 155.8899 85.2779) (end 155.8899 87.9371) (width 0.25) (layer F.Cu) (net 11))
 (segment (start 155.1051 84.4931) (end 155.8899 85.2779) (width 0.25) (layer F.Cu) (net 11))
 (segment (start 156.3899 87.9371) (end 156.3899 84.3809) (width 0.25) (layer F.Cu) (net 12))
 (segment (start 156.0195 81.423) (end 156.9212 80.5213) (width 0.25) (layer F.Cu) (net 12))
 (segment (start 156.0195 84.0105) (end 156.0195 81.423) (width 0.25) (layer F.Cu) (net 12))
 (segment (start 156.3899 84.3809) (end 156.0195 84.0105) (width 0.25) (layer F.Cu) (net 12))
 (segment (start 156.9212 82.5213) (end 156.9212 87.9058) (width 0.25) (layer F.Cu) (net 13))
 (segment (start 156.9212 87.9058) (end 156.8899 87.9371) (width 0.25) (layer F.Cu) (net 13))
 (segment (start 157.3899 87.9371) (end 157.3899 83.9101) (width 0.25) (layer F.Cu) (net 14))
 (segment (start 157.7975 81.4738) (end 158.75 80.5213) (width 0.25) (layer F.Cu) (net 14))
 (segment (start 157.7975 83.5025) (end 157.7975 81.4738) (width 0.25) (layer F.Cu) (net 14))
 (segment (start 157.3899 83.9101) (end 157.7975 83.5025) (width 0.25) (layer F.Cu) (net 14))
 (segment (start 160.5788 82.5213) (end 160.5788 83.5787) (width 0.25) (layer F.Cu) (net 15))
 (segment (start 157.8899 84.9341) (end 157.8899 87.9371) (width 0.25) (layer F.Cu) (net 15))
 (segment (start 159.004 83.82) (end 157.8899 84.9341) (width 0.25) (layer F.Cu) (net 15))
 (segment (start 160.3375 83.82) (end 159.004 83.82) (width 0.25) (layer F.Cu) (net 15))
 (segment (start 160.5788 83.5787) (end 160.3375 83.82) (width 0.25) (layer F.Cu) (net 15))
 (segment (start 158.3899 87.9371) (end 158.3899 85.1961) (width 0.25) (layer F.Cu) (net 16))
 (segment (start 162.3949 83.3501) (end 162.3949 82.5086) (width 0.25) (layer F.Cu) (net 16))
 (segment (start 162.179 83.566) (end 162.3949 83.3501) (width 0.25) (layer F.Cu) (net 16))
 (segment (start 161.417 83.566) (end 162.179 83.566) (width 0.25) (layer F.Cu) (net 16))
 (segment (start 160.7185 84.2645) (end 161.417 83.566) (width 0.25) (layer F.Cu) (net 16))
 (segment (start 159.3215 84.2645) (end 160.7185 84.2645) (width 0.25) (layer F.Cu) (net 16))
 (segment (start 158.3899 85.1961) (end 159.3215 84.2645) (width 0.25) (layer F.Cu) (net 16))
 (segment (start 158.8899 87.9371) (end 158.8899 85.3946) (width 0.25) (layer F.Cu) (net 17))
 (segment (start 164.1856 83.4009) (end 164.1856 82.5086) (width 0.25) (layer F.Cu) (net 17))
 (segment (start 163.5125 84.074) (end 164.1856 83.4009) (width 0.25) (layer F.Cu) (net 17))
 (segment (start 161.6075 84.074) (end 163.5125 84.074) (width 0.25) (layer F.Cu) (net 17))
 (segment (start 160.909 84.7725) (end 161.6075 84.074) (width 0.25) (layer F.Cu) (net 17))
 (segment (start 159.512 84.7725) (end 160.909 84.7725) (width 0.25) (layer F.Cu) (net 17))
 (segment (start 158.8899 85.3946) (end 159.512 84.7725) (width 0.25) (layer F.Cu) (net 17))
 (segment (start 159.3899 87.9371) (end 159.3899 85.9741) (width 0.25) (layer F.Cu) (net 18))
 (segment (start 165.9636 84.1629) (end 165.9636 82.5086) (width 0.25) (layer F.Cu) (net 18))
 (segment (start 165.608 84.5185) (end 165.9636 84.1629) (width 0.25) (layer F.Cu) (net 18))
 (segment (start 161.925 84.5185) (end 165.608 84.5185) (width 0.25) (layer F.Cu) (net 18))
 (segment (start 160.9725 85.471) (end 161.925 84.5185) (width 0.25) (layer F.Cu) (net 18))
 (segment (start 159.893 85.471) (end 160.9725 85.471) (width 0.25) (layer F.Cu) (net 18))
 (segment (start 159.3899 85.9741) (end 159.893 85.471) (width 0.25) (layer F.Cu) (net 18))
 (segment (start 163.6395 70.726) (end 163.6525 70.726) (width 0.25) (layer F.Cu) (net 19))
 (segment (start 163.6525 70.726) (end 165.359502 69.018998) (width 0.25) (layer F.Cu) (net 19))
 (segment (start 173.482 86.2203) (end 170.0403 89.662) (width 0.25) (layer F.Cu) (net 19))
 (segment (start 173.482 77.724) (end 173.482 86.2203) (width 0.25) (layer F.Cu) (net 19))
 (segment (start 171.323 75.565) (end 173.482 77.724) (width 0.25) (layer F.Cu) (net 19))
 (segment (start 171.323 70.0405) (end 171.323 75.565) (width 0.25) (layer F.Cu) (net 19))
 (segment (start 170.301498 69.018998) (end 171.323 70.0405) (width 0.25) (layer F.Cu) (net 19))
 (segment (start 165.359502 69.018998) (end 170.301498 69.018998) (width 0.25) (layer F.Cu) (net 19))
 (segment (start 163.6395 70.726) (end 163.6395 70.4215) (width 0.25) (layer F.Cu) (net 19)))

